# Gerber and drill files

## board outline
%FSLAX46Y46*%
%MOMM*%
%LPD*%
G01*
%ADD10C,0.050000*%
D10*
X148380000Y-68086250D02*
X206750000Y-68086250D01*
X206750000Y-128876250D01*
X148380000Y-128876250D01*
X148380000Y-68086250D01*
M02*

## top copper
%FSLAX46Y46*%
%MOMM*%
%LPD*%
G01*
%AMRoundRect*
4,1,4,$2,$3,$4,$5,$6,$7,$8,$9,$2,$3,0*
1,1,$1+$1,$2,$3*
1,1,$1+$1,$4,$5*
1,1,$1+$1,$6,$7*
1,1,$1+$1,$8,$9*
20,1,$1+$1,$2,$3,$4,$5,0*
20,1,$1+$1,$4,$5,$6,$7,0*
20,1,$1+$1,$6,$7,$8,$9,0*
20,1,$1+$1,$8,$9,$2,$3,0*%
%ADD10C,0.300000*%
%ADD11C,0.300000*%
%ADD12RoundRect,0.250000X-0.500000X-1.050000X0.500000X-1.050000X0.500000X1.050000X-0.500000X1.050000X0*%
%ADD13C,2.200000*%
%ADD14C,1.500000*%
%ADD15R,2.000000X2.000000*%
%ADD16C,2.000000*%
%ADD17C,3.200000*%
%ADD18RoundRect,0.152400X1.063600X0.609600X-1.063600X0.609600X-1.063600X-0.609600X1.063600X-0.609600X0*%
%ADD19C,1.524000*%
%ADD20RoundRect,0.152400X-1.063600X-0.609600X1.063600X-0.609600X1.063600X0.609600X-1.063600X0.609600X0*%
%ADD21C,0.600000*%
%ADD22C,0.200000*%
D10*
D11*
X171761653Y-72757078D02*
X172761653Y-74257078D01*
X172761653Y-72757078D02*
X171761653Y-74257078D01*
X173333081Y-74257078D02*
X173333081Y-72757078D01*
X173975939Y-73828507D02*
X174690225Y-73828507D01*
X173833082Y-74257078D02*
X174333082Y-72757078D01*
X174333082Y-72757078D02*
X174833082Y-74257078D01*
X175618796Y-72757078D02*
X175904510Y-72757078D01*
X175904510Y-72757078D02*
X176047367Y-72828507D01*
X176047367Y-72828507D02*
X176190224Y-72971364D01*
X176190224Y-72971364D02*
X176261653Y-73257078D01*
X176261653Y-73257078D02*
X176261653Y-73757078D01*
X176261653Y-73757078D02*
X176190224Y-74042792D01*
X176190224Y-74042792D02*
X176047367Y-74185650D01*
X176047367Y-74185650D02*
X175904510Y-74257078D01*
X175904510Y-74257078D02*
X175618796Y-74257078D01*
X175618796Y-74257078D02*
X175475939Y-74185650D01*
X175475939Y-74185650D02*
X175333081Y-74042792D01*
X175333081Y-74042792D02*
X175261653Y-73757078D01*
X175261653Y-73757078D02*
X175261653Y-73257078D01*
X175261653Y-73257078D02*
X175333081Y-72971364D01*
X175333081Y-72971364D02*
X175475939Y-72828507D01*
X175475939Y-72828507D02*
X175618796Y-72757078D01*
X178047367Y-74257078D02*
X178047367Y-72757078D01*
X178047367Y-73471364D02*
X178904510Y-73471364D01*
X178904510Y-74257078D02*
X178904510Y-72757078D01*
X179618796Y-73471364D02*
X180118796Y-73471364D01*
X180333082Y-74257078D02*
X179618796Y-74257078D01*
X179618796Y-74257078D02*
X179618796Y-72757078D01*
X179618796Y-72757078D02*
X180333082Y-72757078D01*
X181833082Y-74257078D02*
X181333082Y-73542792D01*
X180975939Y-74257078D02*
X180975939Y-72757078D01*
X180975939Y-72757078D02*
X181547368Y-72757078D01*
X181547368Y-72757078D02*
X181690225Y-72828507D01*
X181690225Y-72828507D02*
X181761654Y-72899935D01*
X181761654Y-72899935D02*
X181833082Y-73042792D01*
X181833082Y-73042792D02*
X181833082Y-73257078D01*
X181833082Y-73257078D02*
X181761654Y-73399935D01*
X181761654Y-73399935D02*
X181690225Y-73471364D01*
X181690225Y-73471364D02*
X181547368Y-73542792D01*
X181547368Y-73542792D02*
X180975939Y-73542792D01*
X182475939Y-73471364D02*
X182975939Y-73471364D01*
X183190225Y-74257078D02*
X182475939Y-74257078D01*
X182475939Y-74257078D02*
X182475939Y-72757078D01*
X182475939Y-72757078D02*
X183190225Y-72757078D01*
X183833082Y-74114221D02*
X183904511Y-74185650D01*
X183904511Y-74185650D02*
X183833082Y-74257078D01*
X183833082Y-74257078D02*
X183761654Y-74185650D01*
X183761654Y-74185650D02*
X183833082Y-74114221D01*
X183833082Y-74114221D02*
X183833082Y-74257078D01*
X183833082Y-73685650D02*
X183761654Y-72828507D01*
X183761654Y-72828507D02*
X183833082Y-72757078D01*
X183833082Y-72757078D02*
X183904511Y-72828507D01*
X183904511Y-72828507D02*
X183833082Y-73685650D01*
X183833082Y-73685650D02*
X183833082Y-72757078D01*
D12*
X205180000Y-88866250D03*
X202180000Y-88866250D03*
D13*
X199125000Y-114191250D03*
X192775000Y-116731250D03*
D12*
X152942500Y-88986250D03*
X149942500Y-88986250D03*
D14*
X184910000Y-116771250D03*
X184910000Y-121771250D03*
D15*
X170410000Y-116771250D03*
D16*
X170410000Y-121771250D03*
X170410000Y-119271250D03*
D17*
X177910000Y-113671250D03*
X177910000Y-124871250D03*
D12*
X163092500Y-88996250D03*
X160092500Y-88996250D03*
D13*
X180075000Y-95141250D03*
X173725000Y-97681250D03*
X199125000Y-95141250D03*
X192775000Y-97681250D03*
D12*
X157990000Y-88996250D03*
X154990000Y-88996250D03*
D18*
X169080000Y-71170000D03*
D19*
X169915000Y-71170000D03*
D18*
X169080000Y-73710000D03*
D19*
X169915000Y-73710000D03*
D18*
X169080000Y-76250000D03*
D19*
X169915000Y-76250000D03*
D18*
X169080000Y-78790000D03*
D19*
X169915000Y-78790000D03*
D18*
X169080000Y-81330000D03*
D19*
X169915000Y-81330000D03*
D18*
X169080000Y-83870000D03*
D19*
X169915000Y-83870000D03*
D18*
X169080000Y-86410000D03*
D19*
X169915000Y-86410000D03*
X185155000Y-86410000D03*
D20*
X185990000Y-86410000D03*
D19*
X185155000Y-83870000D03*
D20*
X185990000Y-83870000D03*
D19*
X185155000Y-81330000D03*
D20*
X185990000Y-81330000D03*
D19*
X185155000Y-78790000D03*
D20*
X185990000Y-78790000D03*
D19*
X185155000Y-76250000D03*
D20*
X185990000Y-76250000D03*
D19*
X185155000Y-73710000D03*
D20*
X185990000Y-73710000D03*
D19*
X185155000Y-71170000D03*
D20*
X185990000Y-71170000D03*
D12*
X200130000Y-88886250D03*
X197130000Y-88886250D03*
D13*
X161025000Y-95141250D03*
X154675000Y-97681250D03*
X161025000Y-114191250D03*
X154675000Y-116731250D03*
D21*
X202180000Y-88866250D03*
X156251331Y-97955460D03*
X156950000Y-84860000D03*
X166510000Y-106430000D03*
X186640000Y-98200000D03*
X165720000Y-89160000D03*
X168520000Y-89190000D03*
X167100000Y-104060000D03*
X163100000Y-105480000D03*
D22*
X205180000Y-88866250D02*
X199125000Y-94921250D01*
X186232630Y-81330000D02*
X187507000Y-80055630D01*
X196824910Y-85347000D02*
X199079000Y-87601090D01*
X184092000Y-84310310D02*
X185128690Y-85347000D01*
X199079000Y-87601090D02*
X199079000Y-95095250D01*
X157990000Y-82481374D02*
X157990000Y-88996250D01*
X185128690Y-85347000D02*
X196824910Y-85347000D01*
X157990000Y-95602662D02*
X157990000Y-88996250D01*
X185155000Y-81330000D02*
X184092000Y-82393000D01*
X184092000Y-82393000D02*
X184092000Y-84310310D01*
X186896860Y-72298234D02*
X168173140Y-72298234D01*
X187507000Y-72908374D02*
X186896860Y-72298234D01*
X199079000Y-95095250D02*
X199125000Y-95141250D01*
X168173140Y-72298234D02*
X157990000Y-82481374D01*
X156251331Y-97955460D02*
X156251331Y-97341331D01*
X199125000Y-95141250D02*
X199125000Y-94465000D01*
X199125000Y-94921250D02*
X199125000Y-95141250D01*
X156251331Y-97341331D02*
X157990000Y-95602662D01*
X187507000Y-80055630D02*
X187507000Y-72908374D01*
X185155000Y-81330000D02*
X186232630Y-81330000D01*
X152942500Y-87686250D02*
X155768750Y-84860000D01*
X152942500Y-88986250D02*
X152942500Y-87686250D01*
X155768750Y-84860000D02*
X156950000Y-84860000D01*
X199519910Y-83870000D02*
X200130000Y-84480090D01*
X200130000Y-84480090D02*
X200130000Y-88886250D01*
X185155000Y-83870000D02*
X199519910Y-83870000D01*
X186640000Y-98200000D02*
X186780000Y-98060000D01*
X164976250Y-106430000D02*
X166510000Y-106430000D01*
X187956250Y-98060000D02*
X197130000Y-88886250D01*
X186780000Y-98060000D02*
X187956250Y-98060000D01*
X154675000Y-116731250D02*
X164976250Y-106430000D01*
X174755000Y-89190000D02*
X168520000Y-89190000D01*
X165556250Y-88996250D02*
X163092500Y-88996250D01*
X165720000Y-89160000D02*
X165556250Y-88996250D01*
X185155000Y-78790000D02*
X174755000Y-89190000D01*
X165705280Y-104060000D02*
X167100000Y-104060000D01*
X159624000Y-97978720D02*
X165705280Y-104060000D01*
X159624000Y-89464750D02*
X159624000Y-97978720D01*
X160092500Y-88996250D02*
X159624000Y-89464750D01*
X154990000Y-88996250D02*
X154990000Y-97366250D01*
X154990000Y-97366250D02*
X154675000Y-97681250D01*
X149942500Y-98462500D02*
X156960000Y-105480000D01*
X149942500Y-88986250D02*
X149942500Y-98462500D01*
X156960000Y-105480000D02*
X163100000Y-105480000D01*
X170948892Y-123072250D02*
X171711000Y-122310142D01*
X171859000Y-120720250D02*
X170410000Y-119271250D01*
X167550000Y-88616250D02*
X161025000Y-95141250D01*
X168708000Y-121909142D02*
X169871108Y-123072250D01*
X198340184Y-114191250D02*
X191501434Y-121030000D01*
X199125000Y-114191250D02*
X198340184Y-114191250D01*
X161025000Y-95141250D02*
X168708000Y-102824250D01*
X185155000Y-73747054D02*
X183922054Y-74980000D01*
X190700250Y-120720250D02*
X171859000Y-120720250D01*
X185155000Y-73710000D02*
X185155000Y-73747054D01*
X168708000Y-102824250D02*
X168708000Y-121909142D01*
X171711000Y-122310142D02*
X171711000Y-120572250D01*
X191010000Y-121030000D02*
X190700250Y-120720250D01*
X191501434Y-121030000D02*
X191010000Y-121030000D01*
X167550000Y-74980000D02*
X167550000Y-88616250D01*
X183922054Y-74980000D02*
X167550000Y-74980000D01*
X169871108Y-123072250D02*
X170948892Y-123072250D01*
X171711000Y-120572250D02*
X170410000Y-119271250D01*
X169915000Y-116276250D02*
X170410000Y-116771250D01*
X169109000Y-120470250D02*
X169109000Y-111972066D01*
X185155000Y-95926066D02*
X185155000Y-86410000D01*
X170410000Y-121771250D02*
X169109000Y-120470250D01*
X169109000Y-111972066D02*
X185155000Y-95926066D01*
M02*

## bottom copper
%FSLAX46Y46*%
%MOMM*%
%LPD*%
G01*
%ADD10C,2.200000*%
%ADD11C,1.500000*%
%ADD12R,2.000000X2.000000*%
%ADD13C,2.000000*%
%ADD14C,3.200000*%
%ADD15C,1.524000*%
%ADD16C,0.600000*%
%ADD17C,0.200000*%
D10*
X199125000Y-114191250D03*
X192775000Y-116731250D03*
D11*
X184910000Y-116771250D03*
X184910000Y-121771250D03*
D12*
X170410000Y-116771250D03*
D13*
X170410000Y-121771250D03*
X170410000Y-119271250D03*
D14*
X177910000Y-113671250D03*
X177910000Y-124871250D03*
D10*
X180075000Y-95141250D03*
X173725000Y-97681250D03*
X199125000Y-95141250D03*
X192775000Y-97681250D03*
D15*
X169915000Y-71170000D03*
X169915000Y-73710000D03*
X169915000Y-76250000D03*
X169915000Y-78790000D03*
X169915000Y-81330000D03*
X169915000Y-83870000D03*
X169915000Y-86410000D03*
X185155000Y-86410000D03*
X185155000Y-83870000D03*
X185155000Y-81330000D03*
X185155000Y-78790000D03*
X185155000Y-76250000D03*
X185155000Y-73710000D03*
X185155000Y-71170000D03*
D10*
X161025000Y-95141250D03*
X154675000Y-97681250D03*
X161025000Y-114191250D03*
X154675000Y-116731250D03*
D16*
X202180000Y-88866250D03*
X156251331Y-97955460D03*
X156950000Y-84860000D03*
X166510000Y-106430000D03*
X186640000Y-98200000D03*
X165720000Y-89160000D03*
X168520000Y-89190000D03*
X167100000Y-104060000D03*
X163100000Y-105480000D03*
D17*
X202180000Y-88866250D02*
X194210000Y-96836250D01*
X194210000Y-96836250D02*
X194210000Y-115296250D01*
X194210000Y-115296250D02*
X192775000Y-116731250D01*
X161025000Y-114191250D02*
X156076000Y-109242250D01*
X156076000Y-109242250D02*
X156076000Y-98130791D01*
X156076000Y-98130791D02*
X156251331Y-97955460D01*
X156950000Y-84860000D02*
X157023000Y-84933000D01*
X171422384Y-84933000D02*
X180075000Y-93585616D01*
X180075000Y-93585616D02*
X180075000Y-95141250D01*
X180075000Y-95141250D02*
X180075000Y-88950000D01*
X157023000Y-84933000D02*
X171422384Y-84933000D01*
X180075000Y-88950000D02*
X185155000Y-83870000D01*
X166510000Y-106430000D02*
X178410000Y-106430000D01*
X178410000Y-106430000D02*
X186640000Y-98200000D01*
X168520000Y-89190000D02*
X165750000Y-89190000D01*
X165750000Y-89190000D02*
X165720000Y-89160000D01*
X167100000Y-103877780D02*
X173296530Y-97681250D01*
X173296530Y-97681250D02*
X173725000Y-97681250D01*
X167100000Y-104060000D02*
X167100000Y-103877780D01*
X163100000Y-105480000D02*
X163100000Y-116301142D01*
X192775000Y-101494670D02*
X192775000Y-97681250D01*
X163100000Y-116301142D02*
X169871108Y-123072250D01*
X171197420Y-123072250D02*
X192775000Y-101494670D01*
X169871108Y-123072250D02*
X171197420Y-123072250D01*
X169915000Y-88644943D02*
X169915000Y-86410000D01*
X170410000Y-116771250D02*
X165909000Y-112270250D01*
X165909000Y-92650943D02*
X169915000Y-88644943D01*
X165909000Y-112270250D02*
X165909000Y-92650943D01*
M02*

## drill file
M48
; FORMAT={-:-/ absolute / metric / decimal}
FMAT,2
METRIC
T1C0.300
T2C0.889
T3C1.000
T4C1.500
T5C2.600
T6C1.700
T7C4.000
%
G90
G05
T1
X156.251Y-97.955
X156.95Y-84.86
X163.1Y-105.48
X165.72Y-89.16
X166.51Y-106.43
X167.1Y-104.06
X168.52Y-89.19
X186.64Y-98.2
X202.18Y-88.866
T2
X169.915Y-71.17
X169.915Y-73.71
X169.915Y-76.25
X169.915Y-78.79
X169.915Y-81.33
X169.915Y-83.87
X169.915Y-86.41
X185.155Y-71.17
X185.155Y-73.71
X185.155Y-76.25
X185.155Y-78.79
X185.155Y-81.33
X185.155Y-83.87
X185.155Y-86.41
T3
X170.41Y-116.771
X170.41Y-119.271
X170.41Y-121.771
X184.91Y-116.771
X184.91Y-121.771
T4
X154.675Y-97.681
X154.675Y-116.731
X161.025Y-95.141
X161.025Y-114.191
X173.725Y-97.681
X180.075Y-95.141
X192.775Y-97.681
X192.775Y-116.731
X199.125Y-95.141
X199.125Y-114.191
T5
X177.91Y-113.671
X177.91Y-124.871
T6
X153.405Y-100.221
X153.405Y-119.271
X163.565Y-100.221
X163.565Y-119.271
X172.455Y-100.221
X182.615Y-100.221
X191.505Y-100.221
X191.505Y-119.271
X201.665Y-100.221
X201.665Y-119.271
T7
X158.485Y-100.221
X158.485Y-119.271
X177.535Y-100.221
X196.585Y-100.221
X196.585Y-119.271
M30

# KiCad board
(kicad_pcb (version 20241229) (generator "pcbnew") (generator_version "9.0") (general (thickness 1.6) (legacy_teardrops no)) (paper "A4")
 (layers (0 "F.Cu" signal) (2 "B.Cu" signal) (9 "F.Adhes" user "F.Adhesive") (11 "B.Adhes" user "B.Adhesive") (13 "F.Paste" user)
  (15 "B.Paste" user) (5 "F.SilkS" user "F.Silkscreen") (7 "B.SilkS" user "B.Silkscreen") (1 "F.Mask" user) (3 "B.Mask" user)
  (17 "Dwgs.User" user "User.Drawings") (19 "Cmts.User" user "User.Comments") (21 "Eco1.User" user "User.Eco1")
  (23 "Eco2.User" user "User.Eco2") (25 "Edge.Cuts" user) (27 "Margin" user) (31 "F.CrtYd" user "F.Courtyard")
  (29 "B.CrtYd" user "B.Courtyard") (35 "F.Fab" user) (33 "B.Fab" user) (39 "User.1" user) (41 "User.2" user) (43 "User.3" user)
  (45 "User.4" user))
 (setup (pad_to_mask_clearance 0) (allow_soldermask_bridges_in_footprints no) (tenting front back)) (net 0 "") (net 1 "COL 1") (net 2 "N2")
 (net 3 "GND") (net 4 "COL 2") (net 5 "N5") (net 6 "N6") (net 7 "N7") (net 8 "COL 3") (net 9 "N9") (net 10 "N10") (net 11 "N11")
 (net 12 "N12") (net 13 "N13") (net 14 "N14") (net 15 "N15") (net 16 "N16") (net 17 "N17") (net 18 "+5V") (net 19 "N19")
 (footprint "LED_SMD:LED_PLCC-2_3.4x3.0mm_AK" (layer "F.Cu") (at 203.68 88.86625)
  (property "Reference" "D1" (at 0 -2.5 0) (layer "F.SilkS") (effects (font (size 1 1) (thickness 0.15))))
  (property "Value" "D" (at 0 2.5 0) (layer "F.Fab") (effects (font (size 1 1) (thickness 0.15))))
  (pad "1" smd roundrect (at 1.5 0) (size 1.5 2.6) (layers "F.Cu" "F.Mask" "F.Paste") (roundrect_rratio 0.1666666667) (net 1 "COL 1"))
  (pad "2" smd roundrect (at -1.5 0) (size 1.5 2.6) (layers "F.Cu" "F.Mask" "F.Paste") (roundrect_rratio 0.1666666667) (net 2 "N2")))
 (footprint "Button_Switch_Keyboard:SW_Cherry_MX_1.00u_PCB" (layer "F.Cu") (at 199.125 114.19125)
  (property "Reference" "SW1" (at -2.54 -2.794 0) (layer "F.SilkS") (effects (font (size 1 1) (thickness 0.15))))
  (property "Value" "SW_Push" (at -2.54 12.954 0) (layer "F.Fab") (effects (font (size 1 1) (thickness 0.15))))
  (pad "" np_thru_hole circle (at -7.62 5.08) (size 1.7 1.7) (drill 1.7) (layers "*.Cu" "*.Mask"))
  (pad "" np_thru_hole circle (at -2.54 5.08) (size 4 4) (drill 4) (layers "*.Cu" "*.Mask"))
  (pad "" np_thru_hole circle (at 2.54 5.08) (size 1.7 1.7) (drill 1.7) (layers "*.Cu" "*.Mask"))
  (pad "1" thru_hole circle (at 0 0) (size 2.2 2.2) (drill 1.5) (layers "*.Cu" "*.Mask") (remove_unused_layers no) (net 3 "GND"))
  (pad "2" thru_hole circle (at -6.35 2.54) (size 2.2 2.2) (drill 1.5) (layers "*.Cu" "*.Mask") (remove_unused_layers no) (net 2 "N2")))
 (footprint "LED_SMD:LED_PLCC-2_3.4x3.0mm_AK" (layer "F.Cu") (at 151.4425 88.98625)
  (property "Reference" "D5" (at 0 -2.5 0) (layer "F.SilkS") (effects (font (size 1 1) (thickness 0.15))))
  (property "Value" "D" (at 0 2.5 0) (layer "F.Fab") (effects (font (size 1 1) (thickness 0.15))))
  (pad "1" smd roundrect (at 1.5 0) (size 1.5 2.6) (layers "F.Cu" "F.Mask" "F.Paste") (roundrect_rratio 0.1666666667) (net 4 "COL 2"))
  (pad "2" smd roundrect (at -1.5 0) (size 1.5 2.6) (layers "F.Cu" "F.Mask" "F.Paste") (roundrect_rratio 0.1666666667) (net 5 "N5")))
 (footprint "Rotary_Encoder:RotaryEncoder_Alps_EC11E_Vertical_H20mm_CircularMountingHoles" (layer "F.Cu") (at 170.41 116.77125)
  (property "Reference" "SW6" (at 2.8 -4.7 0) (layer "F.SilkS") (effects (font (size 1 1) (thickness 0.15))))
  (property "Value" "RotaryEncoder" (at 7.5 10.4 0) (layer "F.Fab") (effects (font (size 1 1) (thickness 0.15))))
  (pad "" thru_hole circle (at 14.5 0) (size 1.5 1.5) (drill 1) (layers "*.Cu" "*.Mask") (remove_unused_layers no))
  (pad "" thru_hole circle (at 14.5 5) (size 1.5 1.5) (drill 1) (layers "*.Cu" "*.Mask") (remove_unused_layers no))
  (pad "A" thru_hole rect (at 0 0) (size 2 2) (drill 1) (layers "*.Cu" "*.Mask") (remove_unused_layers no) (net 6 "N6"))
  (pad "B" thru_hole circle (at 0 5) (size 2 2) (drill 1) (layers "*.Cu" "*.Mask") (remove_unused_layers no) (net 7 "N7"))
  (pad "C" thru_hole circle (at 0 2.5) (size 2 2) (drill 1) (layers "*.Cu" "*.Mask") (remove_unused_layers no) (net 3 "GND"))
  (pad "MP" thru_hole circle (at 7.5 -3.1) (size 3.2 3.2) (drill 2.6) (layers "*.Cu" "*.Mask") (remove_unused_layers no))
  (pad "MP" thru_hole circle (at 7.5 8.1) (size 3.2 3.2) (drill 2.6) (layers "*.Cu" "*.Mask") (remove_unused_layers no)))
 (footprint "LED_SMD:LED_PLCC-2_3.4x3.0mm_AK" (layer "F.Cu") (at 161.5925 88.99625)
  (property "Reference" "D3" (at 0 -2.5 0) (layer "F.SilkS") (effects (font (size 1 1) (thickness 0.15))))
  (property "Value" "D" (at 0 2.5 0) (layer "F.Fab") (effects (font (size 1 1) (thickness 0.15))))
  (pad "1" smd roundrect (at 1.5 0) (size 1.5 2.6) (layers "F.Cu" "F.Mask" "F.Paste") (roundrect_rratio 0.1666666667) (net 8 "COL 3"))
  (pad "2" smd roundrect (at -1.5 0) (size 1.5 2.6) (layers "F.Cu" "F.Mask" "F.Paste") (roundrect_rratio 0.1666666667) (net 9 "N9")))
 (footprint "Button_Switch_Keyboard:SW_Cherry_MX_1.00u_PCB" (layer "F.Cu") (at 180.075 95.14125)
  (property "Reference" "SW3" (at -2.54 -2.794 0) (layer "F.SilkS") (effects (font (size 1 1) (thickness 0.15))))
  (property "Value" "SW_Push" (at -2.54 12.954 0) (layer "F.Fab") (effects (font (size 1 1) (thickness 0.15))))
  (pad "" np_thru_hole circle (at -7.62 5.08) (size 1.7 1.7) (drill 1.7) (layers "*.Cu" "*.Mask"))
  (pad "" np_thru_hole circle (at -2.54 5.08) (size 4 4) (drill 4) (layers "*.Cu" "*.Mask"))
  (pad "" np_thru_hole circle (at 2.54 5.08) (size 1.7 1.7) (drill 1.7) (layers "*.Cu" "*.Mask"))
  (pad "1" thru_hole circle (at 0 0) (size 2.2 2.2) (drill 1.5) (layers "*.Cu" "*.Mask") (remove_unused_layers no) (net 4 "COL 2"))
  (pad "2" thru_hole circle (at -6.35 2.54) (size 2.2 2.2) (drill 1.5) (layers "*.Cu" "*.Mask") (remove_unused_layers no) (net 9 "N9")))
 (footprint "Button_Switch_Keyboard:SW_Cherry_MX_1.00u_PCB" (layer "F.Cu") (at 199.125 95.14125)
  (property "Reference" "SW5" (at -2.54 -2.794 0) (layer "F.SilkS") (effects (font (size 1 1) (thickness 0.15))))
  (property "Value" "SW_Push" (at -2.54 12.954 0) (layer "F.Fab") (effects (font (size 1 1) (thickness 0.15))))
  (pad "" np_thru_hole circle (at -7.62 5.08) (size 1.7 1.7) (drill 1.7) (layers "*.Cu" "*.Mask"))
  (pad "" np_thru_hole circle (at -2.54 5.08) (size 4 4) (drill 4) (layers "*.Cu" "*.Mask"))
  (pad "" np_thru_hole circle (at 2.54 5.08) (size 1.7 1.7) (drill 1.7) (layers "*.Cu" "*.Mask"))
  (pad "1" thru_hole circle (at 0 0) (size 2.2 2.2) (drill 1.5) (layers "*.Cu" "*.Mask") (remove_unused_layers no) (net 1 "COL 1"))
  (pad "2" thru_hole circle (at -6.35 2.54) (size 2.2 2.2) (drill 1.5) (layers "*.Cu" "*.Mask") (remove_unused_layers no) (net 5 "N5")))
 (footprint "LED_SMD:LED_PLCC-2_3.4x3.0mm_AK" (layer "F.Cu") (at 156.49 88.99625)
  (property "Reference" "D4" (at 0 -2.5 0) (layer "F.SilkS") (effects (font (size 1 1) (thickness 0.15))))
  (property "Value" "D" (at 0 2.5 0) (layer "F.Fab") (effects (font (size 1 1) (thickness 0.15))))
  (pad "1" smd roundrect (at 1.5 0) (size 1.5 2.6) (layers "F.Cu" "F.Mask" "F.Paste") (roundrect_rratio 0.1666666667) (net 1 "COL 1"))
  (pad "2" smd roundrect (at -1.5 0) (size 1.5 2.6) (layers "F.Cu" "F.Mask" "F.Paste") (roundrect_rratio 0.1666666667) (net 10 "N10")))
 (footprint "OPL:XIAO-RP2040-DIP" (layer "F.Cu") (at 177.535 78.79)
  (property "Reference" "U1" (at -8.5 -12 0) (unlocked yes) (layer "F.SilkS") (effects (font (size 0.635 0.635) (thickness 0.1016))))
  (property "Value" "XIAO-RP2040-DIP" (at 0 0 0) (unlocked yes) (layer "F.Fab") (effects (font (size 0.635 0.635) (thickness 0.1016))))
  (pad "1" smd roundrect (at -8.455 -7.62 180) (size 2.432 1.524) (layers "F.Cu" "F.Mask") (roundrect_rratio 0.1) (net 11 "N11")
   (thermal_bridge_angle 45))
  (pad "1" thru_hole circle (at -7.62 -7.62 180) (size 1.524 1.524) (drill 0.889) (layers "*.Cu" "*.Mask") (remove_unused_layers no)
   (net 11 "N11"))
  (pad "2" smd roundrect (at -8.455 -5.08 180) (size 2.432 1.524) (layers "F.Cu" "F.Mask") (roundrect_rratio 0.1) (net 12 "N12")
   (thermal_bridge_angle 45))
  (pad "2" thru_hole circle (at -7.62 -5.08 180) (size 1.524 1.524) (drill 0.889) (layers "*.Cu" "*.Mask") (remove_unused_layers no)
   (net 12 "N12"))
  (pad "3" smd roundrect (at -8.455 -2.54 180) (size 2.432 1.524) (layers "F.Cu" "F.Mask") (roundrect_rratio 0.1) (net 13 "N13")
   (thermal_bridge_angle 45))
  (pad "3" thru_hole circle (at -7.62 -2.54 180) (size 1.524 1.524) (drill 0.889) (layers "*.Cu" "*.Mask") (remove_unused_layers no)
   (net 13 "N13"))
  (pad "4" smd roundrect (at -8.455 0 180) (size 2.432 1.524) (layers "F.Cu" "F.Mask") (roundrect_rratio 0.1) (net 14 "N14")
   (thermal_bridge_angle 45))
  (pad "4" thru_hole circle (at -7.62 0 180) (size 1.524 1.524) (drill 0.889) (layers "*.Cu" "*.Mask") (remove_unused_layers no)
   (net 14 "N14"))
  (pad "5" smd roundrect (at -8.455 2.54 180) (size 2.432 1.524) (layers "F.Cu" "F.Mask") (roundrect_rratio 0.1) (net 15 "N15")
   (thermal_bridge_angle 45))
  (pad "5" thru_hole circle (at -7.62 2.54 180) (size 1.524 1.524) (drill 0.889) (layers "*.Cu" "*.Mask") (remove_unused_layers no)
   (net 15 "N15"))
  (pad "6" smd roundrect (at -8.455 5.08 180) (size 2.432 1.524) (layers "F.Cu" "F.Mask") (roundrect_rratio 0.1) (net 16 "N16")
   (thermal_bridge_angle 45))
  (pad "6" thru_hole circle (at -7.62 5.08 180) (size 1.524 1.524) (drill 0.889) (layers "*.Cu" "*.Mask") (remove_unused_layers no)
   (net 16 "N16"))
  (pad "7" smd roundrect (at -8.455 7.62 180) (size 2.432 1.524) (layers "F.Cu" "F.Mask") (roundrect_rratio 0.1) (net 6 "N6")
   (thermal_bridge_angle 45))
  (pad "7" thru_hole circle (at -7.62 7.62 180) (size 1.524 1.524) (drill 0.889) (layers "*.Cu" "*.Mask") (remove_unused_layers no)
   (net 6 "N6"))
  (pad "8" thru_hole circle (at 7.62 7.62) (size 1.524 1.524) (drill 0.889) (layers "*.Cu" "*.Mask") (remove_unused_layers no) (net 7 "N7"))
  (pad "8" smd roundrect (at 8.455 7.62) (size 2.432 1.524) (layers "F.Cu" "F.Mask") (roundrect_rratio 0.1) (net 7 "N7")
   (thermal_bridge_angle 45))
  (pad "9" thru_hole circle (at 7.62 5.08) (size 1.524 1.524) (drill 0.889) (layers "*.Cu" "*.Mask") (remove_unused_layers no)
   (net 4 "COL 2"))
  (pad "9" smd roundrect (at 8.455 5.08) (size 2.432 1.524) (layers "F.Cu" "F.Mask") (roundrect_rratio 0.1) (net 4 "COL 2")
   (thermal_bridge_angle 45))
  (pad "10" thru_hole circle (at 7.62 2.54) (size 1.524 1.524) (drill 0.889) (layers "*.Cu" "*.Mask") (remove_unused_layers no)
   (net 1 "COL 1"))
  (pad "10" smd roundrect (at 8.455 2.54) (size 2.432 1.524) (layers "F.Cu" "F.Mask") (roundrect_rratio 0.1) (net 1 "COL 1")
   (thermal_bridge_angle 45))
  (pad "11" thru_hole circle (at 7.62 0) (size 1.524 1.524) (drill 0.889) (layers "*.Cu" "*.Mask") (remove_unused_layers no) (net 8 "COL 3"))
  (pad "11" smd roundrect (at 8.455 0) (size 2.432 1.524) (layers "F.Cu" "F.Mask") (roundrect_rratio 0.1) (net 8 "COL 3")
   (thermal_bridge_angle 45))
  (pad "12" thru_hole circle (at 7.62 -2.54) (size 1.524 1.524) (drill 0.889) (layers "*.Cu" "*.Mask") (remove_unused_layers no)
   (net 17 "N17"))
  (pad "12" smd roundrect (at 8.455 -2.54) (size 2.432 1.524) (layers "F.Cu" "F.Mask") (roundrect_rratio 0.1) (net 17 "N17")
   (thermal_bridge_angle 45))
  (pad "13" thru_hole circle (at 7.62 -5.08) (size 1.524 1.524) (drill 0.889) (layers "*.Cu" "*.Mask") (remove_unused_layers no)
   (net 3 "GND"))
  (pad "13" smd roundrect (at 8.455 -5.08) (size 2.432 1.524) (layers "F.Cu" "F.Mask") (roundrect_rratio 0.1) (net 3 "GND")
   (thermal_bridge_angle 45))
  (pad "14" thru_hole circle (at 7.62 -7.62) (size 1.524 1.524) (drill 0.889) (layers "*.Cu" "*.Mask") (remove_unused_layers no)
   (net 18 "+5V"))
  (pad "14" smd roundrect (at 8.455 -7.62) (size 2.432 1.524) (layers "F.Cu" "F.Mask") (roundrect_rratio 0.1) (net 18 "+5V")
   (thermal_bridge_angle 45)))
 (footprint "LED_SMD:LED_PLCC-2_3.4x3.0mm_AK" (layer "F.Cu") (at 198.63 88.88625)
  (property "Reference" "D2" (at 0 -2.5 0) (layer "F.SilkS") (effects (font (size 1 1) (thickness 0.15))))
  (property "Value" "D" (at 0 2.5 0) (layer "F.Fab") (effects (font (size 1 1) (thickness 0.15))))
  (pad "1" smd roundrect (at 1.5 0) (size 1.5 2.6) (layers "F.Cu" "F.Mask" "F.Paste") (roundrect_rratio 0.1666666667) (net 4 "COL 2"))
  (pad "2" smd roundrect (at -1.5 0) (size 1.5 2.6) (layers "F.Cu" "F.Mask" "F.Paste") (roundrect_rratio 0.1666666667) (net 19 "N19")))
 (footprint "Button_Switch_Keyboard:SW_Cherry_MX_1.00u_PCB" (layer "F.Cu") (at 161.025 95.14125)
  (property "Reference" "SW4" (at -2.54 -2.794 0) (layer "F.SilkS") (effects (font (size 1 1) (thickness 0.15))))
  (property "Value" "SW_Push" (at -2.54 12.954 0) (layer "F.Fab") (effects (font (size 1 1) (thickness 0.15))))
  (pad "" np_thru_hole circle (at -7.62 5.08) (size 1.7 1.7) (drill 1.7) (layers "*.Cu" "*.Mask"))
  (pad "" np_thru_hole circle (at -2.54 5.08) (size 4 4) (drill 4) (layers "*.Cu" "*.Mask"))
  (pad "" np_thru_hole circle (at 2.54 5.08) (size 1.7 1.7) (drill 1.7) (layers "*.Cu" "*.Mask"))
  (pad "1" thru_hole circle (at 0 0) (size 2.2 2.2) (drill 1.5) (layers "*.Cu" "*.Mask") (remove_unused_layers no) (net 3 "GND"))
  (pad "2" thru_hole circle (at -6.35 2.54) (size 2.2 2.2) (drill 1.5) (layers "*.Cu" "*.Mask") (remove_unused_layers no) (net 10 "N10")))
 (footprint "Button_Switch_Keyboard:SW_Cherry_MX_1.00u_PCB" (layer "F.Cu") (at 161.025 114.19125)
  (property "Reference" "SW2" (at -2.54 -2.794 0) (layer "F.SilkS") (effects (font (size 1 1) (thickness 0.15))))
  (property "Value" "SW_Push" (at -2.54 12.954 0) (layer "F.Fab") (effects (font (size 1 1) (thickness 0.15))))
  (pad "" np_thru_hole circle (at -7.62 5.08) (size 1.7 1.7) (drill 1.7) (layers "*.Cu" "*.Mask"))
  (pad "" np_thru_hole circle (at -2.54 5.08) (size 4 4) (drill 4) (layers "*.Cu" "*.Mask"))
  (pad "" np_thru_hole circle (at 2.54 5.08) (size 1.7 1.7) (drill 1.7) (layers "*.Cu" "*.Mask"))
  (pad "1" thru_hole circle (at 0 0) (size 2.2 2.2) (drill 1.5) (layers "*.Cu" "*.Mask") (remove_unused_layers no) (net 1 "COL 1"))
  (pad "2" thru_hole circle (at -6.35 2.54) (size 2.2 2.2) (drill 1.5) (layers "*.Cu" "*.Mask") (remove_unused_layers no) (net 19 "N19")))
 (gr_rect (start 148.38 68.08625) (end 206.75 128.87625) (stroke (width 0.05) (type default)) (fill no) (layer "Edge.Cuts"))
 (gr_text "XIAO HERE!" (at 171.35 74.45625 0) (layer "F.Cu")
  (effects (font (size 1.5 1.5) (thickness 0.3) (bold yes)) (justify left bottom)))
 (via (at 202.18 88.86625) (size 0.6) (drill 0.3) (layers "F.Cu" "B.Cu") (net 2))
 (segment (start 202.18 88.86625) (end 194.21 96.83625) (width 0.2) (layer "B.Cu") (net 2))
 (segment (start 194.21 96.83625) (end 194.21 115.29625) (width 0.2) (layer "B.Cu") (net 2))
 (segment (start 194.21 115.29625) (end 192.775 116.73125) (width 0.2) (layer "B.Cu") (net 2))
 (segment (start 205.18 88.86625) (end 199.125 94.92125) (width 0.2) (layer "F.Cu") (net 1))
 (segment (start 186.23263 81.33) (end 187.507 80.05563) (width 0.2) (layer "F.Cu") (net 1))
 (segment (start 196.82491 85.347) (end 199.079 87.60109) (width 0.2) (layer "F.Cu") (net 1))
 (segment (start 184.092 84.31031) (end 185.12869 85.347) (width 0.2) (layer "F.Cu") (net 1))
 (segment (start 199.079 87.60109) (end 199.079 95.09525) (width 0.2) (layer "F.Cu") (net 1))
 (segment (start 157.99 82.481374) (end 157.99 88.99625) (width 0.2) (layer "F.Cu") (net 1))
 (segment (start 185.12869 85.347) (end 196.82491 85.347) (width 0.2) (layer "F.Cu") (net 1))
 (segment (start 157.99 95.602662) (end 157.99 88.99625) (width 0.2) (layer "F.Cu") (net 1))
 (segment (start 185.155 81.33) (end 184.092 82.393) (width 0.2) (layer "F.Cu") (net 1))
 (segment (start 184.092 82.393) (end 184.092 84.31031) (width 0.2) (layer "F.Cu") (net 1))
 (segment (start 186.89686 72.298234) (end 168.17314 72.298234) (width 0.2) (layer "F.Cu") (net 1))
 (segment (start 187.507 72.908374) (end 186.89686 72.298234) (width 0.2) (layer "F.Cu") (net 1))
 (segment (start 199.079 95.09525) (end 199.125 95.14125) (width 0.2) (layer "F.Cu") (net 1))
 (segment (start 168.17314 72.298234) (end 157.99 82.481374) (width 0.2) (layer "F.Cu") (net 1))
 (segment (start 156.251331 97.95546) (end 156.251331 97.341331) (width 0.2) (layer "F.Cu") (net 1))
 (segment (start 199.125 95.14125) (end 199.125 94.465) (width 0.2) (layer "F.Cu") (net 1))
 (segment (start 199.125 94.92125) (end 199.125 95.14125) (width 0.2) (layer "F.Cu") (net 1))
 (segment (start 156.251331 97.341331) (end 157.99 95.602662) (width 0.2) (layer "F.Cu") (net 1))
 (segment (start 187.507 80.05563) (end 187.507 72.908374) (width 0.2) (layer "F.Cu") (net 1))
 (segment (start 185.155 81.33) (end 186.23263 81.33) (width 0.2) (layer "F.Cu") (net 1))
 (via (at 156.251331 97.95546) (size 0.6) (drill 0.3) (layers "F.Cu" "B.Cu") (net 1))
 (segment (start 161.025 114.19125) (end 156.076 109.24225) (width 0.2) (layer "B.Cu") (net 1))
 (segment (start 156.076 109.24225) (end 156.076 98.130791) (width 0.2) (layer "B.Cu") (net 1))
 (segment (start 156.076 98.130791) (end 156.251331 97.95546) (width 0.2) (layer "B.Cu") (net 1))
 (segment (start 152.9425 87.68625) (end 155.76875 84.86) (width 0.2) (layer "F.Cu") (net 4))
 (segment (start 152.9425 88.98625) (end 152.9425 87.68625) (width 0.2) (layer "F.Cu") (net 4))
 (segment (start 155.76875 84.86) (end 156.95 84.86) (width 0.2) (layer "F.Cu") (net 4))
 (segment (start 199.51991 83.87) (end 200.13 84.48009) (width 0.2) (layer "F.Cu") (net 4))
 (segment (start 200.13 84.48009) (end 200.13 88.88625) (width 0.2) (layer "F.Cu") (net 4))
 (segment (start 185.155 83.87) (end 199.51991 83.87) (width 0.2) (layer "F.Cu") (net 4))
 (via (at 156.95 84.86) (size 0.6) (drill 0.3) (layers "F.Cu" "B.Cu") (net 4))
 (segment (start 156.95 84.86) (end 157.023 84.933) (width 0.2) (layer "B.Cu") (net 4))
 (segment (start 171.422384 84.933) (end 180.075 93.585616) (width 0.2) (layer "B.Cu") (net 4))
 (segment (start 180.075 93.585616) (end 180.075 95.14125) (width 0.2) (layer "B.Cu") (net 4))
 (segment (start 180.075 95.14125) (end 180.075 88.95) (width 0.2) (layer "B.Cu") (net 4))
 (segment (start 157.023 84.933) (end 171.422384 84.933) (width 0.2) (layer "B.Cu") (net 4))
 (segment (start 180.075 88.95) (end 185.155 83.87) (width 0.2) (layer "B.Cu") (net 4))
 (segment (start 186.64 98.2) (end 186.78 98.06) (width 0.2) (layer "F.Cu") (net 19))
 (segment (start 164.97625 106.43) (end 166.51 106.43) (width 0.2) (layer "F.Cu") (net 19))
 (segment (start 187.95625 98.06) (end 197.13 88.88625) (width 0.2) (layer "F.Cu") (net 19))
 (segment (start 186.78 98.06) (end 187.95625 98.06) (width 0.2) (layer "F.Cu") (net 19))
 (segment (start 154.675 116.73125) (end 164.97625 106.43) (width 0.2) (layer "F.Cu") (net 19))
 (via (at 166.51 106.43) (size 0.6) (drill 0.3) (layers "F.Cu" "B.Cu") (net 19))
 (via (at 186.64 98.2) (size 0.6) (drill 0.3) (layers "F.Cu" "B.Cu") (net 19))
 (segment (start 166.51 106.43) (end 178.41 106.43) (width 0.2) (layer "B.Cu") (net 19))
 (segment (start 178.41 106.43) (end 186.64 98.2) (width 0.2) (layer "B.Cu") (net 19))
 (segment (start 174.755 89.19) (end 168.52 89.19) (width 0.2) (layer "F.Cu") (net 8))
 (segment (start 165.55625 88.99625) (end 163.0925 88.99625) (width 0.2) (layer "F.Cu") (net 8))
 (segment (start 165.72 89.16) (end 165.55625 88.99625) (width 0.2) (layer "F.Cu") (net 8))
 (segment (start 185.155 78.79) (end 174.755 89.19) (width 0.2) (layer "F.Cu") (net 8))
 (via (at 165.72 89.16) (size 0.6) (drill 0.3) (layers "F.Cu" "B.Cu") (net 8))
 (via (at 168.52 89.19) (size 0.6) (drill 0.3) (layers "F.Cu" "B.Cu") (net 8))
 (segment (start 168.52 89.19) (end 165.75 89.19) (width 0.2) (layer "B.Cu") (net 8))
 (segment (start 165.75 89.19) (end 165.72 89.16) (width 0.2) (layer "B.Cu") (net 8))
 (segment (start 165.70528 104.06) (end 167.1 104.06) (width 0.2) (layer "F.Cu") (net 9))
 (segment (start 159.624 97.97872) (end 165.70528 104.06) (width 0.2) (layer "F.Cu") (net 9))
 (segment (start 159.624 89.46475) (end 159.624 97.97872) (width 0.2) (layer "F.Cu") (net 9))
 (segment (start 160.0925 88.99625) (end 159.624 89.46475) (width 0.2) (layer "F.Cu") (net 9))
 (via (at 167.1 104.06) (size 0.6) (drill 0.3) (layers "F.Cu" "B.Cu") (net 9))
 (segment (start 167.1 103.87778) (end 173.29653 97.68125) (width 0.2) (layer "B.Cu") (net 9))
 (segment (start 173.29653 97.68125) (end 173.725 97.68125) (width 0.2) (layer "B.Cu") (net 9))
 (segment (start 167.1 104.06) (end 167.1 103.87778) (width 0.2) (layer "B.Cu") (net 9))
 (segment (start 154.99 88.99625) (end 154.99 97.36625) (width 0.2) (layer "F.Cu") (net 10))
 (segment (start 154.99 97.36625) (end 154.675 97.68125) (width 0.2) (layer "F.Cu") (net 10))
 (segment (start 149.9425 98.4625) (end 156.96 105.48) (width 0.2) (layer "F.Cu") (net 5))
 (segment (start 149.9425 88.98625) (end 149.9425 98.4625) (width 0.2) (layer "F.Cu") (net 5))
 (segment (start 156.96 105.48) (end 163.1 105.48) (width 0.2) (layer "F.Cu") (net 5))
 (via (at 163.1 105.48) (size 0.6) (drill 0.3) (layers "F.Cu" "B.Cu") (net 5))
 (segment (start 163.1 105.48) (end 163.1 116.301142) (width 0.2) (layer "B.Cu") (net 5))
 (segment (start 192.775 101.49467) (end 192.775 97.68125) (width 0.2) (layer "B.Cu") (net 5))
 (segment (start 163.1 116.301142) (end 169.871108 123.07225) (width 0.2) (layer "B.Cu") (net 5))
 (segment (start 171.19742 123.07225) (end 192.775 101.49467) (width 0.2) (layer "B.Cu") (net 5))
 (segment (start 169.871108 123.07225) (end 171.19742 123.07225) (width 0.2) (layer "B.Cu") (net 5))
 (segment (start 170.948892 123.07225) (end 171.711 122.310142) (width 0.2) (layer "F.Cu") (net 3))
 (segment (start 171.859 120.72025) (end 170.41 119.27125) (width 0.2) (layer "F.Cu") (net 3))
 (segment (start 167.55 88.61625) (end 161.025 95.14125) (width 0.2) (layer "F.Cu") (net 3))
 (segment (start 168.708 121.909142) (end 169.871108 123.07225) (width 0.2) (layer "F.Cu") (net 3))
 (segment (start 198.340184 114.19125) (end 191.501434 121.03) (width 0.2) (layer "F.Cu") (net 3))
 (segment (start 199.125 114.19125) (end 198.340184 114.19125) (width 0.2) (layer "F.Cu") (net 3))
 (segment (start 161.025 95.14125) (end 168.708 102.82425) (width 0.2) (layer "F.Cu") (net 3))
 (segment (start 185.155 73.747054) (end 183.922054 74.98) (width 0.2) (layer "F.Cu") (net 3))
 (segment (start 190.70025 120.72025) (end 171.859 120.72025) (width 0.2) (layer "F.Cu") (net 3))
 (segment (start 185.155 73.71) (end 185.155 73.747054) (width 0.2) (layer "F.Cu") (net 3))
 (segment (start 168.708 102.82425) (end 168.708 121.909142) (width 0.2) (layer "F.Cu") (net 3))
 (segment (start 171.711 122.310142) (end 171.711 120.57225) (width 0.2) (layer "F.Cu") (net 3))
 (segment (start 191.01 121.03) (end 190.70025 120.72025) (width 0.2) (layer "F.Cu") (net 3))
 (segment (start 191.501434 121.03) (end 191.01 121.03) (width 0.2) (layer "F.Cu") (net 3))
 (segment (start 167.55 74.98) (end 167.55 88.61625) (width 0.2) (layer "F.Cu") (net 3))
 (segment (start 183.922054 74.98) (end 167.55 74.98) (width 0.2) (layer "F.Cu") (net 3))
 (segment (start 169.871108 123.07225) (end 170.948892 123.07225) (width 0.2) (layer "F.Cu") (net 3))
 (segment (start 171.711 120.57225) (end 170.41 119.27125) (width 0.2) (layer "F.Cu") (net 3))
 (segment (start 169.915 116.27625) (end 170.41 116.77125) (width 0.2) (layer "F.Cu") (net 6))
 (segment (start 169.915 88.644943) (end 169.915 86.41) (width 0.2) (layer "B.Cu") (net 6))
 (segment (start 170.41 116.77125) (end 165.909 112.27025) (width 0.2) (layer "B.Cu") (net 6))
 (segment (start 165.909 92.650943) (end 169.915 88.644943) (width 0.2) (layer "B.Cu") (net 6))
 (segment (start 165.909 112.27025) (end 165.909 92.650943) (width 0.2) (layer "B.Cu") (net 6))
 (segment (start 169.109 120.47025) (end 169.109 111.972066) (width 0.2) (layer "F.Cu") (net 7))
 (segment (start 185.155 95.926066) (end 185.155 86.41) (width 0.2) (layer "F.Cu") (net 7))
 (segment (start 170.41 121.77125) (end 169.109 120.47025) (width 0.2) (layer "F.Cu") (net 7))
 (segment (start 169.109 111.972066) (end 185.155 95.926066) (width 0.2) (layer "F.Cu") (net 7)))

